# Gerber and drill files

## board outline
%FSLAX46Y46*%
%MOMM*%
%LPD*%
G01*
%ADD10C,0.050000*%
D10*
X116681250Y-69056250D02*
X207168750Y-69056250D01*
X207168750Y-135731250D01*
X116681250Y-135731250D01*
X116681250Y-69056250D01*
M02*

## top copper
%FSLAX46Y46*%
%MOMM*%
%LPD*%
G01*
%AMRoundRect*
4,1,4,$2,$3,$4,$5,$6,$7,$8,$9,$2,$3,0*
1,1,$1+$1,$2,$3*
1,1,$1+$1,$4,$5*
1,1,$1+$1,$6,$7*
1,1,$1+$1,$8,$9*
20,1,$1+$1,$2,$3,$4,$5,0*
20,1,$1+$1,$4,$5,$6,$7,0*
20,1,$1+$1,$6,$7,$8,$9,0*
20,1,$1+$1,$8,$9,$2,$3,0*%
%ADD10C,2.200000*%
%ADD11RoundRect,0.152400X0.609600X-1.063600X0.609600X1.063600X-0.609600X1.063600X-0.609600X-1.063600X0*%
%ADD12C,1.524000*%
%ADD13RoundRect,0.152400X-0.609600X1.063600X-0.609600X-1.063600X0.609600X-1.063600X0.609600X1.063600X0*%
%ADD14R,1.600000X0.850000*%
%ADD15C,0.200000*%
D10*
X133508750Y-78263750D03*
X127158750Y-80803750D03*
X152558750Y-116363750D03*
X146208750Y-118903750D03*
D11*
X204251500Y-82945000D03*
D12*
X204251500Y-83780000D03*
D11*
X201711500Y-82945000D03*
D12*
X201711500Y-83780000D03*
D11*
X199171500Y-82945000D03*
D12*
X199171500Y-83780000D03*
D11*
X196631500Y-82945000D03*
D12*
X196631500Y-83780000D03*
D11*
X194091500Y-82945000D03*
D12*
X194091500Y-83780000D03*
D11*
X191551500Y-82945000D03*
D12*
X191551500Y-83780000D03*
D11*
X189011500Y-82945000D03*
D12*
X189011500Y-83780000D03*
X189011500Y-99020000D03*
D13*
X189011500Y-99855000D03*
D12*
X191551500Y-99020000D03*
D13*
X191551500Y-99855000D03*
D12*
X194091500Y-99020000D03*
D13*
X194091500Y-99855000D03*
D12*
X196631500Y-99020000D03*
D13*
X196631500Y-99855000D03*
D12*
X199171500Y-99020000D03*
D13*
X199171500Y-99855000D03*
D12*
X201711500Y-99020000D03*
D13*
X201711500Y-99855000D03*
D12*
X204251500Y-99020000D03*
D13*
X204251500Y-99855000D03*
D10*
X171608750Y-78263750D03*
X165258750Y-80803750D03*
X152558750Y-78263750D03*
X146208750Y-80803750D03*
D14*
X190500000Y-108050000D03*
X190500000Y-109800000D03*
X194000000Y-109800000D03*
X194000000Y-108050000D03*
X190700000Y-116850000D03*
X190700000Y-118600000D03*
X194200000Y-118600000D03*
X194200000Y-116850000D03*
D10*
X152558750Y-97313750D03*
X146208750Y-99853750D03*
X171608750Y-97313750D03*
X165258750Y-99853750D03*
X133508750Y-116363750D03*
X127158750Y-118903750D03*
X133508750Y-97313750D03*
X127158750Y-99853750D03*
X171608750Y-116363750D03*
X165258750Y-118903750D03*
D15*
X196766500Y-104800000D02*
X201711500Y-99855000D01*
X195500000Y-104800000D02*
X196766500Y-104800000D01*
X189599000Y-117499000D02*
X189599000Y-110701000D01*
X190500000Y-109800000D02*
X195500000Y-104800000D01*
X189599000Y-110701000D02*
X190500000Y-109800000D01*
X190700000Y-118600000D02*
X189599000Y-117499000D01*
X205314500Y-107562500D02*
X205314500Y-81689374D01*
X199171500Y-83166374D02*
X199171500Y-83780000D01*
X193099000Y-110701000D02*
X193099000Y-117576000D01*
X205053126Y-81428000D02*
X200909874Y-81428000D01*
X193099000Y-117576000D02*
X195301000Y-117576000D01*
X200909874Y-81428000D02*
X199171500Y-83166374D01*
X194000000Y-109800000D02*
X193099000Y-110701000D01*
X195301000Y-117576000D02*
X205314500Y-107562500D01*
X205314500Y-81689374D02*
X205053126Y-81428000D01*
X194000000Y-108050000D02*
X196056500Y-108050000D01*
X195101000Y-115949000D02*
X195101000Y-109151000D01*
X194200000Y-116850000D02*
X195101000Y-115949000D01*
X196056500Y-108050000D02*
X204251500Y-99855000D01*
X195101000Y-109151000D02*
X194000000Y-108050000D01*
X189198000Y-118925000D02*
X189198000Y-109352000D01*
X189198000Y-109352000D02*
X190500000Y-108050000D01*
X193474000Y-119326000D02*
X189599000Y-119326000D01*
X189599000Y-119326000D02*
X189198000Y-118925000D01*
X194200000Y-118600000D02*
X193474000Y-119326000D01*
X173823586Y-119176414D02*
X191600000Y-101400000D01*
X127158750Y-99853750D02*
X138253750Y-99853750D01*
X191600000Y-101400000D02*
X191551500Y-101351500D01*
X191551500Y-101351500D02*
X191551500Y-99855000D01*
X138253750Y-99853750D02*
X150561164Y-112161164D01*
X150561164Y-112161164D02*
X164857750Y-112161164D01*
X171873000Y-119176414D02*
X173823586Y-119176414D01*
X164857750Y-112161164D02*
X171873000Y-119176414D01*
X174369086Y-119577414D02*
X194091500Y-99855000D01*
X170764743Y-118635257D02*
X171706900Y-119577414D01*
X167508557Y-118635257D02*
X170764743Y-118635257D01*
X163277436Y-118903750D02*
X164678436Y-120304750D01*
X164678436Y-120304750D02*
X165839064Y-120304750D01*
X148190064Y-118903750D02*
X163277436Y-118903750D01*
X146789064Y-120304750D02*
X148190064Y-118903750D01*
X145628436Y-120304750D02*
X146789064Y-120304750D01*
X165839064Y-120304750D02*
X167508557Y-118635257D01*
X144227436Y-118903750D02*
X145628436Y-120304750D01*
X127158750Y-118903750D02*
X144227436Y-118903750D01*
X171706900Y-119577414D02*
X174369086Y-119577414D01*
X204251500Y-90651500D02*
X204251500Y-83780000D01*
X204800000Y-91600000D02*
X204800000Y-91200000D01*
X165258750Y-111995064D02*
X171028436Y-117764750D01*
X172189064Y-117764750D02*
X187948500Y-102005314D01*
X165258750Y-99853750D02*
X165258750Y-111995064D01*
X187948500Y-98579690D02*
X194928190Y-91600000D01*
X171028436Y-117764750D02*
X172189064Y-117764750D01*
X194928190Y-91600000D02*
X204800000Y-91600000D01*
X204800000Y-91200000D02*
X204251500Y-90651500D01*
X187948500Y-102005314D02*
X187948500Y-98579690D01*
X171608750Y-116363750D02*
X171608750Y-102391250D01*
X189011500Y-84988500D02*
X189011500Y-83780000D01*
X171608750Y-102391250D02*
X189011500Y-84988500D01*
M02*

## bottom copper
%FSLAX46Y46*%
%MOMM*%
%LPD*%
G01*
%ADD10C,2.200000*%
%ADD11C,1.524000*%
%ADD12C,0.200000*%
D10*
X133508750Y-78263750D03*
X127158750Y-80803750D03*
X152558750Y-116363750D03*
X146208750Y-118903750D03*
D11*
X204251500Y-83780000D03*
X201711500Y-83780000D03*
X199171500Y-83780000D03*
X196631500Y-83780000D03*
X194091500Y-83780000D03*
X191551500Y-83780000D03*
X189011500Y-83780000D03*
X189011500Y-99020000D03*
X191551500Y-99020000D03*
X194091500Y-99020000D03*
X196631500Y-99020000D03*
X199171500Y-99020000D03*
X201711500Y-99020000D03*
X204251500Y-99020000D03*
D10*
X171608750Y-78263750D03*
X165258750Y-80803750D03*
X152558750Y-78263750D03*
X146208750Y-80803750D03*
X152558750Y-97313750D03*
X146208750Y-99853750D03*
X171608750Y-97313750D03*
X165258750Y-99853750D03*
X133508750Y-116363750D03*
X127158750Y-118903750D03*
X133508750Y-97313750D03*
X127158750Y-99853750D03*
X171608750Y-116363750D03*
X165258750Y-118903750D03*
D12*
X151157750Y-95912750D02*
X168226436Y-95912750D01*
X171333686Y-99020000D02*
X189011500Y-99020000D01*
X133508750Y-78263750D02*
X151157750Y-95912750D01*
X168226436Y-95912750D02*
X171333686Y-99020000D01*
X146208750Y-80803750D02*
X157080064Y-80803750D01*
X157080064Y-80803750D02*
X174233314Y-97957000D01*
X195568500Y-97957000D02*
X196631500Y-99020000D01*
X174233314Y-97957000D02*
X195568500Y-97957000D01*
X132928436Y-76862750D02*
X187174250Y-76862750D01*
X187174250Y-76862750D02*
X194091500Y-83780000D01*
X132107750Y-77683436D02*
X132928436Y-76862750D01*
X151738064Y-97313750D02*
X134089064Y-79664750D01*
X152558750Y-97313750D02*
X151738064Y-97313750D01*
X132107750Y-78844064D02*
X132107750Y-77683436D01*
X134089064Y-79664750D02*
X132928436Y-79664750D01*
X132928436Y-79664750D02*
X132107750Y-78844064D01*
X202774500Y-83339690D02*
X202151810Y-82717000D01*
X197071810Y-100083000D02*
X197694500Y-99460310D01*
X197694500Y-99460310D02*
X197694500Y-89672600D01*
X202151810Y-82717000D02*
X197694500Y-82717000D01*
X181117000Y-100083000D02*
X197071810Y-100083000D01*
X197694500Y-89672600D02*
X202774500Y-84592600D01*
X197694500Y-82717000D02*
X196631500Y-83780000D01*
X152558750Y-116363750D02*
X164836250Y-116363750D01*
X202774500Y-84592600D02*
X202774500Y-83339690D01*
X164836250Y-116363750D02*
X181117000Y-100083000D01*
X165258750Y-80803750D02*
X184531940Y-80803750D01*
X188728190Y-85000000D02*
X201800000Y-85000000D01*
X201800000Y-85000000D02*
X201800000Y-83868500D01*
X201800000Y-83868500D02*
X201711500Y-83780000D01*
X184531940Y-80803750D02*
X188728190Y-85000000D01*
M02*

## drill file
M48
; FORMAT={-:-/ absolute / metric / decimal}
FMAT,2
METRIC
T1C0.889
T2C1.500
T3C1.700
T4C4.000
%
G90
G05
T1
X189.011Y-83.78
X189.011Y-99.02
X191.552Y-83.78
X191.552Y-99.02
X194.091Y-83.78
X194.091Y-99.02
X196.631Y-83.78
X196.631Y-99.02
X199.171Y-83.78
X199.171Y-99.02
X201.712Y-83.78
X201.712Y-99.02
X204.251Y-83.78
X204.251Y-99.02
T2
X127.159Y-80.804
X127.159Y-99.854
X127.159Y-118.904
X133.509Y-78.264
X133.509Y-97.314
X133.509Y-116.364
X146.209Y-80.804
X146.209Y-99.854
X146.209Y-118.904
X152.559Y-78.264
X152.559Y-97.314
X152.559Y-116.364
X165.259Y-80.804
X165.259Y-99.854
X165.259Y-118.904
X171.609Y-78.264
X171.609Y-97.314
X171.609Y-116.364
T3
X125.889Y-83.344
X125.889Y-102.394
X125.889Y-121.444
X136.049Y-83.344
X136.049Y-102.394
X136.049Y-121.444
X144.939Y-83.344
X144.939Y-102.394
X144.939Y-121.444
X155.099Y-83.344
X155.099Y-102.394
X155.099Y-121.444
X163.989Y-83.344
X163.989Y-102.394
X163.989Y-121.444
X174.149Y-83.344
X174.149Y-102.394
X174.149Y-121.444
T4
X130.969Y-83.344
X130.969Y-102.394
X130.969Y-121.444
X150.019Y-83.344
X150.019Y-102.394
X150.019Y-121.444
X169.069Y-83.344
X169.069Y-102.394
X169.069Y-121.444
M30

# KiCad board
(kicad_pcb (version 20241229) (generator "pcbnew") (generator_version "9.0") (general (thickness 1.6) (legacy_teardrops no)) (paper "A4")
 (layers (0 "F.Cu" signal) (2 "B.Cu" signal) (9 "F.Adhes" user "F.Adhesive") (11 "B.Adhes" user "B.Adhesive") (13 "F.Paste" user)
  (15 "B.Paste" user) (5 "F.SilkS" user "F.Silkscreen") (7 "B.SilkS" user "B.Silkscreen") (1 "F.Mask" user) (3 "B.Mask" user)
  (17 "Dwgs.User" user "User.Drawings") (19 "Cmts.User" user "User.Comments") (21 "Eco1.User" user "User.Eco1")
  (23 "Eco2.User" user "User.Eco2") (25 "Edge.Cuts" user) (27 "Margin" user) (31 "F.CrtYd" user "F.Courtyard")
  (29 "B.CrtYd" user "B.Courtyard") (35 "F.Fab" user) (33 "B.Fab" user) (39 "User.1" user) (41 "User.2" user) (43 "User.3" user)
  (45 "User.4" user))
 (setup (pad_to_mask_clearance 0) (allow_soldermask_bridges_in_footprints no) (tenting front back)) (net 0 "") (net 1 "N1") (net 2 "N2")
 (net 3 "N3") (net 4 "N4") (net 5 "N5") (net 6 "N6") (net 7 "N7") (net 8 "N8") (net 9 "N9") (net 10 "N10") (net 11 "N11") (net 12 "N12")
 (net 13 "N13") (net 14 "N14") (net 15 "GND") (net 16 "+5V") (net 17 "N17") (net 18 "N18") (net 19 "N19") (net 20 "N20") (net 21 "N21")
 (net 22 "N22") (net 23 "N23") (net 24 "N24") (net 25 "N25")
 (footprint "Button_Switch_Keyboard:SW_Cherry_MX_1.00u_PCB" (layer "F.Cu") (at 133.50875 78.26375)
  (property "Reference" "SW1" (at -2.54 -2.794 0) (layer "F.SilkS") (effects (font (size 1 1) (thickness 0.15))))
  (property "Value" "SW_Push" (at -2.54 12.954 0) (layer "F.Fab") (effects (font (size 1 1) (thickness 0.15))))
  (pad "" np_thru_hole circle (at -7.62 5.08) (size 1.7 1.7) (drill 1.7) (layers "*.Cu" "*.Mask"))
  (pad "" np_thru_hole circle (at -2.54 5.08) (size 4 4) (drill 4) (layers "*.Cu" "*.Mask"))
  (pad "" np_thru_hole circle (at 2.54 5.08) (size 1.7 1.7) (drill 1.7) (layers "*.Cu" "*.Mask"))
  (pad "1" thru_hole circle (at 0 0) (size 2.2 2.2) (drill 1.5) (layers "*.Cu" "*.Mask") (remove_unused_layers no) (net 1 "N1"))
  (pad "2" thru_hole circle (at -6.35 2.54) (size 2.2 2.2) (drill 1.5) (layers "*.Cu" "*.Mask") (remove_unused_layers no) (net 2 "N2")))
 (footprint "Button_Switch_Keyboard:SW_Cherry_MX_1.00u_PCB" (layer "F.Cu") (at 152.55875 116.36375)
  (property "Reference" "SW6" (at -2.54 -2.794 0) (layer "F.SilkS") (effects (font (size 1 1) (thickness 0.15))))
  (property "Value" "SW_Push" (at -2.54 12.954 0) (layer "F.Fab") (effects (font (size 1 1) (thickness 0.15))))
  (pad "" np_thru_hole circle (at -7.62 5.08) (size 1.7 1.7) (drill 1.7) (layers "*.Cu" "*.Mask"))
  (pad "" np_thru_hole circle (at -2.54 5.08) (size 4 4) (drill 4) (layers "*.Cu" "*.Mask"))
  (pad "" np_thru_hole circle (at 2.54 5.08) (size 1.7 1.7) (drill 1.7) (layers "*.Cu" "*.Mask"))
  (pad "1" thru_hole circle (at 0 0) (size 2.2 2.2) (drill 1.5) (layers "*.Cu" "*.Mask") (remove_unused_layers no) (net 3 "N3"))
  (pad "2" thru_hole circle (at -6.35 2.54) (size 2.2 2.2) (drill 1.5) (layers "*.Cu" "*.Mask") (remove_unused_layers no) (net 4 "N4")))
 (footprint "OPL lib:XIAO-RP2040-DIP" (layer "F.Cu") (at 196.6315 91.4 -90)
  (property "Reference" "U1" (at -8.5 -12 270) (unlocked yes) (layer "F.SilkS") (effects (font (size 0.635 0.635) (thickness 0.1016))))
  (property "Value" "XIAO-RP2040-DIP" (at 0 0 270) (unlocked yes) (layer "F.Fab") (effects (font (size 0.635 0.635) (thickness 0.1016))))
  (pad "1" smd roundrect (at -8.455 -7.62 90) (size 2.432 1.524) (layers "F.Cu" "F.Mask") (roundrect_rratio 0.1) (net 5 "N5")
   (thermal_bridge_angle 45))
  (pad "1" thru_hole circle (at -7.62 -7.62 90) (size 1.524 1.524) (drill 0.889) (layers "*.Cu" "*.Mask") (remove_unused_layers no)
   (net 5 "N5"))
  (pad "2" smd roundrect (at -8.455 -5.08 90) (size 2.432 1.524) (layers "F.Cu" "F.Mask") (roundrect_rratio 0.1) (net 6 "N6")
   (thermal_bridge_angle 45))
  (pad "2" thru_hole circle (at -7.62 -5.08 90) (size 1.524 1.524) (drill 0.889) (layers "*.Cu" "*.Mask") (remove_unused_layers no)
   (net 6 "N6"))
  (pad "3" smd roundrect (at -8.455 -2.54 90) (size 2.432 1.524) (layers "F.Cu" "F.Mask") (roundrect_rratio 0.1) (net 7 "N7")
   (thermal_bridge_angle 45))
  (pad "3" thru_hole circle (at -7.62 -2.54 90) (size 1.524 1.524) (drill 0.889) (layers "*.Cu" "*.Mask") (remove_unused_layers no)
   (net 7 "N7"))
  (pad "4" smd roundrect (at -8.455 0 90) (size 2.432 1.524) (layers "F.Cu" "F.Mask") (roundrect_rratio 0.1) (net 3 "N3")
   (thermal_bridge_angle 45))
  (pad "4" thru_hole circle (at -7.62 0 90) (size 1.524 1.524) (drill 0.889) (layers "*.Cu" "*.Mask") (remove_unused_layers no) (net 3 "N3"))
  (pad "5" smd roundrect (at -8.455 2.54 90) (size 2.432 1.524) (layers "F.Cu" "F.Mask") (roundrect_rratio 0.1) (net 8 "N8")
   (thermal_bridge_angle 45))
  (pad "5" thru_hole circle (at -7.62 2.54 90) (size 1.524 1.524) (drill 0.889) (layers "*.Cu" "*.Mask") (remove_unused_layers no)
   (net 8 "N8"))
  (pad "6" smd roundrect (at -8.455 5.08 90) (size 2.432 1.524) (layers "F.Cu" "F.Mask") (roundrect_rratio 0.1) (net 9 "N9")
   (thermal_bridge_angle 45))
  (pad "6" thru_hole circle (at -7.62 5.08 90) (size 1.524 1.524) (drill 0.889) (layers "*.Cu" "*.Mask") (remove_unused_layers no)
   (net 9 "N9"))
  (pad "7" smd roundrect (at -8.455 7.62 90) (size 2.432 1.524) (layers "F.Cu" "F.Mask") (roundrect_rratio 0.1) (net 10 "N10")
   (thermal_bridge_angle 45))
  (pad "7" thru_hole circle (at -7.62 7.62 90) (size 1.524 1.524) (drill 0.889) (layers "*.Cu" "*.Mask") (remove_unused_layers no)
   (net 10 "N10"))
  (pad "8" thru_hole circle (at 7.62 7.62 270) (size 1.524 1.524) (drill 0.889) (layers "*.Cu" "*.Mask") (remove_unused_layers no)
   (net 1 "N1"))
  (pad "8" smd roundrect (at 8.455 7.62 270) (size 2.432 1.524) (layers "F.Cu" "F.Mask") (roundrect_rratio 0.1) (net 1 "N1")
   (thermal_bridge_angle 45))
  (pad "9" thru_hole circle (at 7.62 5.08 270) (size 1.524 1.524) (drill 0.889) (layers "*.Cu" "*.Mask") (remove_unused_layers no)
   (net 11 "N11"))
  (pad "9" smd roundrect (at 8.455 5.08 270) (size 2.432 1.524) (layers "F.Cu" "F.Mask") (roundrect_rratio 0.1) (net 11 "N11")
   (thermal_bridge_angle 45))
  (pad "10" thru_hole circle (at 7.62 2.54 270) (size 1.524 1.524) (drill 0.889) (layers "*.Cu" "*.Mask") (remove_unused_layers no)
   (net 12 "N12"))
  (pad "10" smd roundrect (at 8.455 2.54 270) (size 2.432 1.524) (layers "F.Cu" "F.Mask") (roundrect_rratio 0.1) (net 12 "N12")
   (thermal_bridge_angle 45))
  (pad "11" thru_hole circle (at 7.62 0 270) (size 1.524 1.524) (drill 0.889) (layers "*.Cu" "*.Mask") (remove_unused_layers no)
   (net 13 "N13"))
  (pad "11" smd roundrect (at 8.455 0 270) (size 2.432 1.524) (layers "F.Cu" "F.Mask") (roundrect_rratio 0.1) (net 13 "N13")
   (thermal_bridge_angle 45))
  (pad "12" thru_hole circle (at 7.62 -2.54 270) (size 1.524 1.524) (drill 0.889) (layers "*.Cu" "*.Mask") (remove_unused_layers no)
   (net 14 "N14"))
  (pad "12" smd roundrect (at 8.455 -2.54 270) (size 2.432 1.524) (layers "F.Cu" "F.Mask") (roundrect_rratio 0.1) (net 14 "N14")
   (thermal_bridge_angle 45))
  (pad "13" thru_hole circle (at 7.62 -5.08 270) (size 1.524 1.524) (drill 0.889) (layers "*.Cu" "*.Mask") (remove_unused_layers no)
   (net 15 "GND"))
  (pad "13" smd roundrect (at 8.455 -5.08 270) (size 2.432 1.524) (layers "F.Cu" "F.Mask") (roundrect_rratio 0.1) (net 15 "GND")
   (thermal_bridge_angle 45))
  (pad "14" thru_hole circle (at 7.62 -7.62 270) (size 1.524 1.524) (drill 0.889) (layers "*.Cu" "*.Mask") (remove_unused_layers no)
   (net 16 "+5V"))
  (pad "14" smd roundrect (at 8.455 -7.62 270) (size 2.432 1.524) (layers "F.Cu" "F.Mask") (roundrect_rratio 0.1) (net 16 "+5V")
   (thermal_bridge_angle 45)))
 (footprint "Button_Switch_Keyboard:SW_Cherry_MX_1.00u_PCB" (layer "F.Cu") (at 171.60875 78.26375)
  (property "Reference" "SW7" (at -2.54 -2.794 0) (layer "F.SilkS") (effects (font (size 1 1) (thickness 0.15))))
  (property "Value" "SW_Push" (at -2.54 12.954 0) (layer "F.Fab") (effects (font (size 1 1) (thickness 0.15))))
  (pad "" np_thru_hole circle (at -7.62 5.08) (size 1.7 1.7) (drill 1.7) (layers "*.Cu" "*.Mask"))
  (pad "" np_thru_hole circle (at -2.54 5.08) (size 4 4) (drill 4) (layers "*.Cu" "*.Mask"))
  (pad "" np_thru_hole circle (at 2.54 5.08) (size 1.7 1.7) (drill 1.7) (layers "*.Cu" "*.Mask"))
  (pad "1" thru_hole circle (at 0 0) (size 2.2 2.2) (drill 1.5) (layers "*.Cu" "*.Mask") (remove_unused_layers no) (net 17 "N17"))
  (pad "2" thru_hole circle (at -6.35 2.54) (size 2.2 2.2) (drill 1.5) (layers "*.Cu" "*.Mask") (remove_unused_layers no) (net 6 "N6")))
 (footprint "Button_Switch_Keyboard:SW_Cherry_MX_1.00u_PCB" (layer "F.Cu") (at 152.55875 78.26375)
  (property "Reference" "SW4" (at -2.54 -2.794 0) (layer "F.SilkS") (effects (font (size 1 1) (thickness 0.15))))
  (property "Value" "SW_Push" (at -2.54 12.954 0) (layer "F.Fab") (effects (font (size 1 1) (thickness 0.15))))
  (pad "" np_thru_hole circle (at -7.62 5.08) (size 1.7 1.7) (drill 1.7) (layers "*.Cu" "*.Mask"))
  (pad "" np_thru_hole circle (at -2.54 5.08) (size 4 4) (drill 4) (layers "*.Cu" "*.Mask"))
  (pad "" np_thru_hole circle (at 2.54 5.08) (size 1.7 1.7) (drill 1.7) (layers "*.Cu" "*.Mask"))
  (pad "1" thru_hole circle (at 0 0) (size 2.2 2.2) (drill 1.5) (layers "*.Cu" "*.Mask") (remove_unused_layers no) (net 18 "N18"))
  (pad "2" thru_hole circle (at -6.35 2.54) (size 2.2 2.2) (drill 1.5) (layers "*.Cu" "*.Mask") (remove_unused_layers no) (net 13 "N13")))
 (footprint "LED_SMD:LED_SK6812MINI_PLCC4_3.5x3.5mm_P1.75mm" (layer "F.Cu") (at 192.25 108.925)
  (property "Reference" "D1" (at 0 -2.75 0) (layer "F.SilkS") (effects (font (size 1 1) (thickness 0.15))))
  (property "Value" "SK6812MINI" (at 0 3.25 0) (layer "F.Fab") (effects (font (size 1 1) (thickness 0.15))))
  (pad "1" smd rect (at -1.75 -0.875) (size 1.6 0.85) (layers "F.Cu" "F.Mask" "F.Paste") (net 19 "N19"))
  (pad "2" smd rect (at -1.75 0.875) (size 1.6 0.85) (layers "F.Cu" "F.Mask" "F.Paste") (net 15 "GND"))
  (pad "3" smd rect (at 1.75 0.875) (size 1.6 0.85) (layers "F.Cu" "F.Mask" "F.Paste") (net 7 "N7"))
  (pad "4" smd rect (at 1.75 -0.875) (size 1.6 0.85) (layers "F.Cu" "F.Mask" "F.Paste") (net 16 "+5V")))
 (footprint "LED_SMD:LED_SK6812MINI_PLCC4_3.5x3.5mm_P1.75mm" (layer "F.Cu") (at 192.45 117.725)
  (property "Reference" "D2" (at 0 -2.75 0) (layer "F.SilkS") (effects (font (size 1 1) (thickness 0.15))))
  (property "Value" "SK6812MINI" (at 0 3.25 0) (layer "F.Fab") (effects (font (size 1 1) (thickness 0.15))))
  (pad "1" smd rect (at -1.75 -0.875) (size 1.6 0.85) (layers "F.Cu" "F.Mask" "F.Paste") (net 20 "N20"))
  (pad "2" smd rect (at -1.75 0.875) (size 1.6 0.85) (layers "F.Cu" "F.Mask" "F.Paste") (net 15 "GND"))
  (pad "3" smd rect (at 1.75 0.875) (size 1.6 0.85) (layers "F.Cu" "F.Mask" "F.Paste") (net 19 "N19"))
  (pad "4" smd rect (at 1.75 -0.875) (size 1.6 0.85) (layers "F.Cu" "F.Mask" "F.Paste") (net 16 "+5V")))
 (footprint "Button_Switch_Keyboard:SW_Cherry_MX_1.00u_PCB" (layer "F.Cu") (at 152.55875 97.31375)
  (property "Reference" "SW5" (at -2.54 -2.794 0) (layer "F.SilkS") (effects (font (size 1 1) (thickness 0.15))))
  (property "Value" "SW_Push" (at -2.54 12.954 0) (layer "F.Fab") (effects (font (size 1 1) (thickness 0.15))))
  (pad "" np_thru_hole circle (at -7.62 5.08) (size 1.7 1.7) (drill 1.7) (layers "*.Cu" "*.Mask"))
  (pad "" np_thru_hole circle (at -2.54 5.08) (size 4 4) (drill 4) (layers "*.Cu" "*.Mask"))
  (pad "" np_thru_hole circle (at 2.54 5.08) (size 1.7 1.7) (drill 1.7) (layers "*.Cu" "*.Mask"))
  (pad "1" thru_hole circle (at 0 0) (size 2.2 2.2) (drill 1.5) (layers "*.Cu" "*.Mask") (remove_unused_layers no) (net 8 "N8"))
  (pad "2" thru_hole circle (at -6.35 2.54) (size 2.2 2.2) (drill 1.5) (layers "*.Cu" "*.Mask") (remove_unused_layers no) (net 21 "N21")))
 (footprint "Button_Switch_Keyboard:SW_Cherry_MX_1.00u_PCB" (layer "F.Cu") (at 171.60875 97.31375)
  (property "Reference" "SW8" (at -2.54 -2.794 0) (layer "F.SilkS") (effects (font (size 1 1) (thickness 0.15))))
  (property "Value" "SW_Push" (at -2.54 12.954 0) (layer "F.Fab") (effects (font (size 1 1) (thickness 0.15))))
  (pad "" np_thru_hole circle (at -7.62 5.08) (size 1.7 1.7) (drill 1.7) (layers "*.Cu" "*.Mask"))
  (pad "" np_thru_hole circle (at -2.54 5.08) (size 4 4) (drill 4) (layers "*.Cu" "*.Mask"))
  (pad "" np_thru_hole circle (at 2.54 5.08) (size 1.7 1.7) (drill 1.7) (layers "*.Cu" "*.Mask"))
  (pad "1" thru_hole circle (at 0 0) (size 2.2 2.2) (drill 1.5) (layers "*.Cu" "*.Mask") (remove_unused_layers no) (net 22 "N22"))
  (pad "2" thru_hole circle (at -6.35 2.54) (size 2.2 2.2) (drill 1.5) (layers "*.Cu" "*.Mask") (remove_unused_layers no) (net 5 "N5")))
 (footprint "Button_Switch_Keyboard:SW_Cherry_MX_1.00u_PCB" (layer "F.Cu") (at 133.50875 116.36375)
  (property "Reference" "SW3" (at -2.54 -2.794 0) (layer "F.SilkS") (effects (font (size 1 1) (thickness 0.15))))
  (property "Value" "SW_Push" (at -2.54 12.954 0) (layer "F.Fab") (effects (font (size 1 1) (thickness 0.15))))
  (pad "" np_thru_hole circle (at -7.62 5.08) (size 1.7 1.7) (drill 1.7) (layers "*.Cu" "*.Mask"))
  (pad "" np_thru_hole circle (at -2.54 5.08) (size 4 4) (drill 4) (layers "*.Cu" "*.Mask"))
  (pad "" np_thru_hole circle (at 2.54 5.08) (size 1.7 1.7) (drill 1.7) (layers "*.Cu" "*.Mask"))
  (pad "1" thru_hole circle (at 0 0) (size 2.2 2.2) (drill 1.5) (layers "*.Cu" "*.Mask") (remove_unused_layers no) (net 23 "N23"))
  (pad "2" thru_hole circle (at -6.35 2.54) (size 2.2 2.2) (drill 1.5) (layers "*.Cu" "*.Mask") (remove_unused_layers no) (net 12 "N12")))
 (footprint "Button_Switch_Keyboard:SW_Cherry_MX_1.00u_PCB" (layer "F.Cu") (at 133.50875 97.31375)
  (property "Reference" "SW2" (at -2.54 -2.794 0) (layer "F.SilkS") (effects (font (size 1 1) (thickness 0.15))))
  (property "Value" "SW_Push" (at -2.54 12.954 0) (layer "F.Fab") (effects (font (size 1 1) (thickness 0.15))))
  (pad "" np_thru_hole circle (at -7.62 5.08) (size 1.7 1.7) (drill 1.7) (layers "*.Cu" "*.Mask"))
  (pad "" np_thru_hole circle (at -2.54 5.08) (size 4 4) (drill 4) (layers "*.Cu" "*.Mask"))
  (pad "" np_thru_hole circle (at 2.54 5.08) (size 1.7 1.7) (drill 1.7) (layers "*.Cu" "*.Mask"))
  (pad "1" thru_hole circle (at 0 0) (size 2.2 2.2) (drill 1.5) (layers "*.Cu" "*.Mask") (remove_unused_layers no) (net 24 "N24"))
  (pad "2" thru_hole circle (at -6.35 2.54) (size 2.2 2.2) (drill 1.5) (layers "*.Cu" "*.Mask") (remove_unused_layers no) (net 11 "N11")))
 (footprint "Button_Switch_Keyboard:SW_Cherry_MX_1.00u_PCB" (layer "F.Cu") (at 171.60875 116.36375)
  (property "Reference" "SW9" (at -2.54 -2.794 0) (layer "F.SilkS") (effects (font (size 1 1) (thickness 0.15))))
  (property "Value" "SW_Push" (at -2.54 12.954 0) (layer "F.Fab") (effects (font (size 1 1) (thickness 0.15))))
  (pad "" np_thru_hole circle (at -7.62 5.08) (size 1.7 1.7) (drill 1.7) (layers "*.Cu" "*.Mask"))
  (pad "" np_thru_hole circle (at -2.54 5.08) (size 4 4) (drill 4) (layers "*.Cu" "*.Mask"))
  (pad "" np_thru_hole circle (at 2.54 5.08) (size 1.7 1.7) (drill 1.7) (layers "*.Cu" "*.Mask"))
  (pad "1" thru_hole circle (at 0 0) (size 2.2 2.2) (drill 1.5) (layers "*.Cu" "*.Mask") (remove_unused_layers no) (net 10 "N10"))
  (pad "2" thru_hole circle (at -6.35 2.54) (size 2.2 2.2) (drill 1.5) (layers "*.Cu" "*.Mask") (remove_unused_layers no) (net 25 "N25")))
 (gr_rect (start 116.68125 69.05625) (end 207.16875 135.73125) (stroke (width 0.05) (type default)) (fill no) (layer "Edge.Cuts"))
 (segment (start 196.7665 104.8) (end 201.7115 99.855) (width 0.2) (layer "F.Cu") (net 15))
 (segment (start 195.5 104.8) (end 196.7665 104.8) (width 0.2) (layer "F.Cu") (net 15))
 (segment (start 189.599 117.499) (end 189.599 110.701) (width 0.2) (layer "F.Cu") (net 15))
 (segment (start 190.5 109.8) (end 195.5 104.8) (width 0.2) (layer "F.Cu") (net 15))
 (segment (start 189.599 110.701) (end 190.5 109.8) (width 0.2) (layer "F.Cu") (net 15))
 (segment (start 190.7 118.6) (end 189.599 117.499) (width 0.2) (layer "F.Cu") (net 15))
 (segment (start 205.3145 107.5625) (end 205.3145 81.689374) (width 0.2) (layer "F.Cu") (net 7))
 (segment (start 199.1715 83.166374) (end 199.1715 83.78) (width 0.2) (layer "F.Cu") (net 7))
 (segment (start 193.099 110.701) (end 193.099 117.576) (width 0.2) (layer "F.Cu") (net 7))
 (segment (start 205.053126 81.428) (end 200.909874 81.428) (width 0.2) (layer "F.Cu") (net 7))
 (segment (start 193.099 117.576) (end 195.301 117.576) (width 0.2) (layer "F.Cu") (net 7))
 (segment (start 200.909874 81.428) (end 199.1715 83.166374) (width 0.2) (layer "F.Cu") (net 7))
 (segment (start 194 109.8) (end 193.099 110.701) (width 0.2) (layer "F.Cu") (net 7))
 (segment (start 195.301 117.576) (end 205.3145 107.5625) (width 0.2) (layer "F.Cu") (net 7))
 (segment (start 205.3145 81.689374) (end 205.053126 81.428) (width 0.2) (layer "F.Cu") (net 7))
 (segment (start 194 108.05) (end 196.0565 108.05) (width 0.2) (layer "F.Cu") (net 16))
 (segment (start 195.101 115.949) (end 195.101 109.151) (width 0.2) (layer "F.Cu") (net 16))
 (segment (start 194.2 116.85) (end 195.101 115.949) (width 0.2) (layer "F.Cu") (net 16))
 (segment (start 196.0565 108.05) (end 204.2515 99.855) (width 0.2) (layer "F.Cu") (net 16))
 (segment (start 195.101 109.151) (end 194 108.05) (width 0.2) (layer "F.Cu") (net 16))
 (segment (start 189.198 118.925) (end 189.198 109.352) (width 0.2) (layer "F.Cu") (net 19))
 (segment (start 189.198 109.352) (end 190.5 108.05) (width 0.2) (layer "F.Cu") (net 19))
 (segment (start 193.474 119.326) (end 189.599 119.326) (width 0.2) (layer "F.Cu") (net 19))
 (segment (start 189.599 119.326) (end 189.198 118.925) (width 0.2) (layer "F.Cu") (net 19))
 (segment (start 194.2 118.6) (end 193.474 119.326) (width 0.2) (layer "F.Cu") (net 19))
 (segment (start 151.15775 95.91275) (end 168.226436 95.91275) (width 0.2) (layer "B.Cu") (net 1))
 (segment (start 171.333686 99.02) (end 189.0115 99.02) (width 0.2) (layer "B.Cu") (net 1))
 (segment (start 133.50875 78.26375) (end 151.15775 95.91275) (width 0.2) (layer "B.Cu") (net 1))
 (segment (start 168.226436 95.91275) (end 171.333686 99.02) (width 0.2) (layer "B.Cu") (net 1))
 (segment (start 173.823586 119.176414) (end 191.6 101.4) (width 0.2) (layer "F.Cu") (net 11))
 (segment (start 127.15875 99.85375) (end 138.25375 99.85375) (width 0.2) (layer "F.Cu") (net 11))
 (segment (start 191.6 101.4) (end 191.5515 101.3515) (width 0.2) (layer "F.Cu") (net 11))
 (segment (start 191.5515 101.3515) (end 191.5515 99.855) (width 0.2) (layer "F.Cu") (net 11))
 (segment (start 138.25375 99.85375) (end 150.561164 112.161164) (width 0.2) (layer "F.Cu") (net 11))
 (segment (start 150.561164 112.161164) (end 164.85775 112.161164) (width 0.2) (layer "F.Cu") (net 11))
 (segment (start 171.873 119.176414) (end 173.823586 119.176414) (width 0.2) (layer "F.Cu") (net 11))
 (segment (start 164.85775 112.161164) (end 171.873 119.176414) (width 0.2) (layer "F.Cu") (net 11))
 (segment (start 174.369086 119.577414) (end 194.0915 99.855) (width 0.2) (layer "F.Cu") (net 12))
 (segment (start 170.764743 118.635257) (end 171.7069 119.577414) (width 0.2) (layer "F.Cu") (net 12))
 (segment (start 167.508557 118.635257) (end 170.764743 118.635257) (width 0.2) (layer "F.Cu") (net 12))
 (segment (start 163.277436 118.90375) (end 164.678436 120.30475) (width 0.2) (layer "F.Cu") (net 12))
 (segment (start 164.678436 120.30475) (end 165.839064 120.30475) (width 0.2) (layer "F.Cu") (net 12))
 (segment (start 148.190064 118.90375) (end 163.277436 118.90375) (width 0.2) (layer "F.Cu") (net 12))
 (segment (start 146.789064 120.30475) (end 148.190064 118.90375) (width 0.2) (layer "F.Cu") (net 12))
 (segment (start 145.628436 120.30475) (end 146.789064 120.30475) (width 0.2) (layer "F.Cu") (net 12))
 (segment (start 165.839064 120.30475) (end 167.508557 118.635257) (width 0.2) (layer "F.Cu") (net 12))
 (segment (start 144.227436 118.90375) (end 145.628436 120.30475) (width 0.2) (layer "F.Cu") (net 12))
 (segment (start 127.15875 118.90375) (end 144.227436 118.90375) (width 0.2) (layer "F.Cu") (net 12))
 (segment (start 171.7069 119.577414) (end 174.369086 119.577414) (width 0.2) (layer "F.Cu") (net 12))
 (segment (start 146.20875 80.80375) (end 157.080064 80.80375) (width 0.2) (layer "B.Cu") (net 13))
 (segment (start 157.080064 80.80375) (end 174.233314 97.957) (width 0.2) (layer "B.Cu") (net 13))
 (segment (start 195.5685 97.957) (end 196.6315 99.02) (width 0.2) (layer "B.Cu") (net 13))
 (segment (start 174.233314 97.957) (end 195.5685 97.957) (width 0.2) (layer "B.Cu") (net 13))
 (segment (start 132.928436 76.86275) (end 187.17425 76.86275) (width 0.2) (layer "B.Cu") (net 8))
 (segment (start 187.17425 76.86275) (end 194.0915 83.78) (width 0.2) (layer "B.Cu") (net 8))
 (segment (start 132.10775 77.683436) (end 132.928436 76.86275) (width 0.2) (layer "B.Cu") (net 8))
 (segment (start 151.738064 97.31375) (end 134.089064 79.66475) (width 0.2) (layer "B.Cu") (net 8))
 (segment (start 152.55875 97.31375) (end 151.738064 97.31375) (width 0.2) (layer "B.Cu") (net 8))
 (segment (start 132.10775 78.844064) (end 132.10775 77.683436) (width 0.2) (layer "B.Cu") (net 8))
 (segment (start 134.089064 79.66475) (end 132.928436 79.66475) (width 0.2) (layer "B.Cu") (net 8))
 (segment (start 132.928436 79.66475) (end 132.10775 78.844064) (width 0.2) (layer "B.Cu") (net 8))
 (segment (start 202.7745 83.33969) (end 202.15181 82.717) (width 0.2) (layer "B.Cu") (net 3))
 (segment (start 197.07181 100.083) (end 197.6945 99.46031) (width 0.2) (layer "B.Cu") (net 3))
 (segment (start 197.6945 99.46031) (end 197.6945 89.6726) (width 0.2) (layer "B.Cu") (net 3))
 (segment (start 202.15181 82.717) (end 197.6945 82.717) (width 0.2) (layer "B.Cu") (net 3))
 (segment (start 181.117 100.083) (end 197.07181 100.083) (width 0.2) (layer "B.Cu") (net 3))
 (segment (start 197.6945 89.6726) (end 202.7745 84.5926) (width 0.2) (layer "B.Cu") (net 3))
 (segment (start 197.6945 82.717) (end 196.6315 83.78) (width 0.2) (layer "B.Cu") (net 3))
 (segment (start 152.55875 116.36375) (end 164.83625 116.36375) (width 0.2) (layer "B.Cu") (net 3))
 (segment (start 202.7745 84.5926) (end 202.7745 83.33969) (width 0.2) (layer "B.Cu") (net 3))
 (segment (start 164.83625 116.36375) (end 181.117 100.083) (width 0.2) (layer "B.Cu") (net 3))
 (segment (start 165.25875 80.80375) (end 184.53194 80.80375) (width 0.2) (layer "B.Cu") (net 6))
 (segment (start 188.72819 85) (end 201.8 85) (width 0.2) (layer "B.Cu") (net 6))
 (segment (start 201.8 85) (end 201.8 83.8685) (width 0.2) (layer "B.Cu") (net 6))
 (segment (start 201.8 83.8685) (end 201.7115 83.78) (width 0.2) (layer "B.Cu") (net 6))
 (segment (start 184.53194 80.80375) (end 188.72819 85) (width 0.2) (layer "B.Cu") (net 6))
 (segment (start 204.2515 90.6515) (end 204.2515 83.78) (width 0.2) (layer "F.Cu") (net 5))
 (segment (start 204.8 91.6) (end 204.8 91.2) (width 0.2) (layer "F.Cu") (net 5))
 (segment (start 165.25875 111.995064) (end 171.028436 117.76475) (width 0.2) (layer "F.Cu") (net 5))
 (segment (start 172.189064 117.76475) (end 187.9485 102.005314) (width 0.2) (layer "F.Cu") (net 5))
 (segment (start 165.25875 99.85375) (end 165.25875 111.995064) (width 0.2) (layer "F.Cu") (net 5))
 (segment (start 187.9485 98.57969) (end 194.92819 91.6) (width 0.2) (layer "F.Cu") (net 5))
 (segment (start 171.028436 117.76475) (end 172.189064 117.76475) (width 0.2) (layer "F.Cu") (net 5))
 (segment (start 194.92819 91.6) (end 204.8 91.6) (width 0.2) (layer "F.Cu") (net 5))
 (segment (start 204.8 91.2) (end 204.2515 90.6515) (width 0.2) (layer "F.Cu") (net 5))
 (segment (start 187.9485 102.005314) (end 187.9485 98.57969) (width 0.2) (layer "F.Cu") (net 5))
 (segment (start 171.60875 116.36375) (end 171.60875 102.39125) (width 0.2) (layer "F.Cu") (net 10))
 (segment (start 189.0115 84.9885) (end 189.0115 83.78) (width 0.2) (layer "F.Cu") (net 10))
 (segment (start 171.60875 102.39125) (end 189.0115 84.9885) (width 0.2) (layer "F.Cu") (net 10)))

